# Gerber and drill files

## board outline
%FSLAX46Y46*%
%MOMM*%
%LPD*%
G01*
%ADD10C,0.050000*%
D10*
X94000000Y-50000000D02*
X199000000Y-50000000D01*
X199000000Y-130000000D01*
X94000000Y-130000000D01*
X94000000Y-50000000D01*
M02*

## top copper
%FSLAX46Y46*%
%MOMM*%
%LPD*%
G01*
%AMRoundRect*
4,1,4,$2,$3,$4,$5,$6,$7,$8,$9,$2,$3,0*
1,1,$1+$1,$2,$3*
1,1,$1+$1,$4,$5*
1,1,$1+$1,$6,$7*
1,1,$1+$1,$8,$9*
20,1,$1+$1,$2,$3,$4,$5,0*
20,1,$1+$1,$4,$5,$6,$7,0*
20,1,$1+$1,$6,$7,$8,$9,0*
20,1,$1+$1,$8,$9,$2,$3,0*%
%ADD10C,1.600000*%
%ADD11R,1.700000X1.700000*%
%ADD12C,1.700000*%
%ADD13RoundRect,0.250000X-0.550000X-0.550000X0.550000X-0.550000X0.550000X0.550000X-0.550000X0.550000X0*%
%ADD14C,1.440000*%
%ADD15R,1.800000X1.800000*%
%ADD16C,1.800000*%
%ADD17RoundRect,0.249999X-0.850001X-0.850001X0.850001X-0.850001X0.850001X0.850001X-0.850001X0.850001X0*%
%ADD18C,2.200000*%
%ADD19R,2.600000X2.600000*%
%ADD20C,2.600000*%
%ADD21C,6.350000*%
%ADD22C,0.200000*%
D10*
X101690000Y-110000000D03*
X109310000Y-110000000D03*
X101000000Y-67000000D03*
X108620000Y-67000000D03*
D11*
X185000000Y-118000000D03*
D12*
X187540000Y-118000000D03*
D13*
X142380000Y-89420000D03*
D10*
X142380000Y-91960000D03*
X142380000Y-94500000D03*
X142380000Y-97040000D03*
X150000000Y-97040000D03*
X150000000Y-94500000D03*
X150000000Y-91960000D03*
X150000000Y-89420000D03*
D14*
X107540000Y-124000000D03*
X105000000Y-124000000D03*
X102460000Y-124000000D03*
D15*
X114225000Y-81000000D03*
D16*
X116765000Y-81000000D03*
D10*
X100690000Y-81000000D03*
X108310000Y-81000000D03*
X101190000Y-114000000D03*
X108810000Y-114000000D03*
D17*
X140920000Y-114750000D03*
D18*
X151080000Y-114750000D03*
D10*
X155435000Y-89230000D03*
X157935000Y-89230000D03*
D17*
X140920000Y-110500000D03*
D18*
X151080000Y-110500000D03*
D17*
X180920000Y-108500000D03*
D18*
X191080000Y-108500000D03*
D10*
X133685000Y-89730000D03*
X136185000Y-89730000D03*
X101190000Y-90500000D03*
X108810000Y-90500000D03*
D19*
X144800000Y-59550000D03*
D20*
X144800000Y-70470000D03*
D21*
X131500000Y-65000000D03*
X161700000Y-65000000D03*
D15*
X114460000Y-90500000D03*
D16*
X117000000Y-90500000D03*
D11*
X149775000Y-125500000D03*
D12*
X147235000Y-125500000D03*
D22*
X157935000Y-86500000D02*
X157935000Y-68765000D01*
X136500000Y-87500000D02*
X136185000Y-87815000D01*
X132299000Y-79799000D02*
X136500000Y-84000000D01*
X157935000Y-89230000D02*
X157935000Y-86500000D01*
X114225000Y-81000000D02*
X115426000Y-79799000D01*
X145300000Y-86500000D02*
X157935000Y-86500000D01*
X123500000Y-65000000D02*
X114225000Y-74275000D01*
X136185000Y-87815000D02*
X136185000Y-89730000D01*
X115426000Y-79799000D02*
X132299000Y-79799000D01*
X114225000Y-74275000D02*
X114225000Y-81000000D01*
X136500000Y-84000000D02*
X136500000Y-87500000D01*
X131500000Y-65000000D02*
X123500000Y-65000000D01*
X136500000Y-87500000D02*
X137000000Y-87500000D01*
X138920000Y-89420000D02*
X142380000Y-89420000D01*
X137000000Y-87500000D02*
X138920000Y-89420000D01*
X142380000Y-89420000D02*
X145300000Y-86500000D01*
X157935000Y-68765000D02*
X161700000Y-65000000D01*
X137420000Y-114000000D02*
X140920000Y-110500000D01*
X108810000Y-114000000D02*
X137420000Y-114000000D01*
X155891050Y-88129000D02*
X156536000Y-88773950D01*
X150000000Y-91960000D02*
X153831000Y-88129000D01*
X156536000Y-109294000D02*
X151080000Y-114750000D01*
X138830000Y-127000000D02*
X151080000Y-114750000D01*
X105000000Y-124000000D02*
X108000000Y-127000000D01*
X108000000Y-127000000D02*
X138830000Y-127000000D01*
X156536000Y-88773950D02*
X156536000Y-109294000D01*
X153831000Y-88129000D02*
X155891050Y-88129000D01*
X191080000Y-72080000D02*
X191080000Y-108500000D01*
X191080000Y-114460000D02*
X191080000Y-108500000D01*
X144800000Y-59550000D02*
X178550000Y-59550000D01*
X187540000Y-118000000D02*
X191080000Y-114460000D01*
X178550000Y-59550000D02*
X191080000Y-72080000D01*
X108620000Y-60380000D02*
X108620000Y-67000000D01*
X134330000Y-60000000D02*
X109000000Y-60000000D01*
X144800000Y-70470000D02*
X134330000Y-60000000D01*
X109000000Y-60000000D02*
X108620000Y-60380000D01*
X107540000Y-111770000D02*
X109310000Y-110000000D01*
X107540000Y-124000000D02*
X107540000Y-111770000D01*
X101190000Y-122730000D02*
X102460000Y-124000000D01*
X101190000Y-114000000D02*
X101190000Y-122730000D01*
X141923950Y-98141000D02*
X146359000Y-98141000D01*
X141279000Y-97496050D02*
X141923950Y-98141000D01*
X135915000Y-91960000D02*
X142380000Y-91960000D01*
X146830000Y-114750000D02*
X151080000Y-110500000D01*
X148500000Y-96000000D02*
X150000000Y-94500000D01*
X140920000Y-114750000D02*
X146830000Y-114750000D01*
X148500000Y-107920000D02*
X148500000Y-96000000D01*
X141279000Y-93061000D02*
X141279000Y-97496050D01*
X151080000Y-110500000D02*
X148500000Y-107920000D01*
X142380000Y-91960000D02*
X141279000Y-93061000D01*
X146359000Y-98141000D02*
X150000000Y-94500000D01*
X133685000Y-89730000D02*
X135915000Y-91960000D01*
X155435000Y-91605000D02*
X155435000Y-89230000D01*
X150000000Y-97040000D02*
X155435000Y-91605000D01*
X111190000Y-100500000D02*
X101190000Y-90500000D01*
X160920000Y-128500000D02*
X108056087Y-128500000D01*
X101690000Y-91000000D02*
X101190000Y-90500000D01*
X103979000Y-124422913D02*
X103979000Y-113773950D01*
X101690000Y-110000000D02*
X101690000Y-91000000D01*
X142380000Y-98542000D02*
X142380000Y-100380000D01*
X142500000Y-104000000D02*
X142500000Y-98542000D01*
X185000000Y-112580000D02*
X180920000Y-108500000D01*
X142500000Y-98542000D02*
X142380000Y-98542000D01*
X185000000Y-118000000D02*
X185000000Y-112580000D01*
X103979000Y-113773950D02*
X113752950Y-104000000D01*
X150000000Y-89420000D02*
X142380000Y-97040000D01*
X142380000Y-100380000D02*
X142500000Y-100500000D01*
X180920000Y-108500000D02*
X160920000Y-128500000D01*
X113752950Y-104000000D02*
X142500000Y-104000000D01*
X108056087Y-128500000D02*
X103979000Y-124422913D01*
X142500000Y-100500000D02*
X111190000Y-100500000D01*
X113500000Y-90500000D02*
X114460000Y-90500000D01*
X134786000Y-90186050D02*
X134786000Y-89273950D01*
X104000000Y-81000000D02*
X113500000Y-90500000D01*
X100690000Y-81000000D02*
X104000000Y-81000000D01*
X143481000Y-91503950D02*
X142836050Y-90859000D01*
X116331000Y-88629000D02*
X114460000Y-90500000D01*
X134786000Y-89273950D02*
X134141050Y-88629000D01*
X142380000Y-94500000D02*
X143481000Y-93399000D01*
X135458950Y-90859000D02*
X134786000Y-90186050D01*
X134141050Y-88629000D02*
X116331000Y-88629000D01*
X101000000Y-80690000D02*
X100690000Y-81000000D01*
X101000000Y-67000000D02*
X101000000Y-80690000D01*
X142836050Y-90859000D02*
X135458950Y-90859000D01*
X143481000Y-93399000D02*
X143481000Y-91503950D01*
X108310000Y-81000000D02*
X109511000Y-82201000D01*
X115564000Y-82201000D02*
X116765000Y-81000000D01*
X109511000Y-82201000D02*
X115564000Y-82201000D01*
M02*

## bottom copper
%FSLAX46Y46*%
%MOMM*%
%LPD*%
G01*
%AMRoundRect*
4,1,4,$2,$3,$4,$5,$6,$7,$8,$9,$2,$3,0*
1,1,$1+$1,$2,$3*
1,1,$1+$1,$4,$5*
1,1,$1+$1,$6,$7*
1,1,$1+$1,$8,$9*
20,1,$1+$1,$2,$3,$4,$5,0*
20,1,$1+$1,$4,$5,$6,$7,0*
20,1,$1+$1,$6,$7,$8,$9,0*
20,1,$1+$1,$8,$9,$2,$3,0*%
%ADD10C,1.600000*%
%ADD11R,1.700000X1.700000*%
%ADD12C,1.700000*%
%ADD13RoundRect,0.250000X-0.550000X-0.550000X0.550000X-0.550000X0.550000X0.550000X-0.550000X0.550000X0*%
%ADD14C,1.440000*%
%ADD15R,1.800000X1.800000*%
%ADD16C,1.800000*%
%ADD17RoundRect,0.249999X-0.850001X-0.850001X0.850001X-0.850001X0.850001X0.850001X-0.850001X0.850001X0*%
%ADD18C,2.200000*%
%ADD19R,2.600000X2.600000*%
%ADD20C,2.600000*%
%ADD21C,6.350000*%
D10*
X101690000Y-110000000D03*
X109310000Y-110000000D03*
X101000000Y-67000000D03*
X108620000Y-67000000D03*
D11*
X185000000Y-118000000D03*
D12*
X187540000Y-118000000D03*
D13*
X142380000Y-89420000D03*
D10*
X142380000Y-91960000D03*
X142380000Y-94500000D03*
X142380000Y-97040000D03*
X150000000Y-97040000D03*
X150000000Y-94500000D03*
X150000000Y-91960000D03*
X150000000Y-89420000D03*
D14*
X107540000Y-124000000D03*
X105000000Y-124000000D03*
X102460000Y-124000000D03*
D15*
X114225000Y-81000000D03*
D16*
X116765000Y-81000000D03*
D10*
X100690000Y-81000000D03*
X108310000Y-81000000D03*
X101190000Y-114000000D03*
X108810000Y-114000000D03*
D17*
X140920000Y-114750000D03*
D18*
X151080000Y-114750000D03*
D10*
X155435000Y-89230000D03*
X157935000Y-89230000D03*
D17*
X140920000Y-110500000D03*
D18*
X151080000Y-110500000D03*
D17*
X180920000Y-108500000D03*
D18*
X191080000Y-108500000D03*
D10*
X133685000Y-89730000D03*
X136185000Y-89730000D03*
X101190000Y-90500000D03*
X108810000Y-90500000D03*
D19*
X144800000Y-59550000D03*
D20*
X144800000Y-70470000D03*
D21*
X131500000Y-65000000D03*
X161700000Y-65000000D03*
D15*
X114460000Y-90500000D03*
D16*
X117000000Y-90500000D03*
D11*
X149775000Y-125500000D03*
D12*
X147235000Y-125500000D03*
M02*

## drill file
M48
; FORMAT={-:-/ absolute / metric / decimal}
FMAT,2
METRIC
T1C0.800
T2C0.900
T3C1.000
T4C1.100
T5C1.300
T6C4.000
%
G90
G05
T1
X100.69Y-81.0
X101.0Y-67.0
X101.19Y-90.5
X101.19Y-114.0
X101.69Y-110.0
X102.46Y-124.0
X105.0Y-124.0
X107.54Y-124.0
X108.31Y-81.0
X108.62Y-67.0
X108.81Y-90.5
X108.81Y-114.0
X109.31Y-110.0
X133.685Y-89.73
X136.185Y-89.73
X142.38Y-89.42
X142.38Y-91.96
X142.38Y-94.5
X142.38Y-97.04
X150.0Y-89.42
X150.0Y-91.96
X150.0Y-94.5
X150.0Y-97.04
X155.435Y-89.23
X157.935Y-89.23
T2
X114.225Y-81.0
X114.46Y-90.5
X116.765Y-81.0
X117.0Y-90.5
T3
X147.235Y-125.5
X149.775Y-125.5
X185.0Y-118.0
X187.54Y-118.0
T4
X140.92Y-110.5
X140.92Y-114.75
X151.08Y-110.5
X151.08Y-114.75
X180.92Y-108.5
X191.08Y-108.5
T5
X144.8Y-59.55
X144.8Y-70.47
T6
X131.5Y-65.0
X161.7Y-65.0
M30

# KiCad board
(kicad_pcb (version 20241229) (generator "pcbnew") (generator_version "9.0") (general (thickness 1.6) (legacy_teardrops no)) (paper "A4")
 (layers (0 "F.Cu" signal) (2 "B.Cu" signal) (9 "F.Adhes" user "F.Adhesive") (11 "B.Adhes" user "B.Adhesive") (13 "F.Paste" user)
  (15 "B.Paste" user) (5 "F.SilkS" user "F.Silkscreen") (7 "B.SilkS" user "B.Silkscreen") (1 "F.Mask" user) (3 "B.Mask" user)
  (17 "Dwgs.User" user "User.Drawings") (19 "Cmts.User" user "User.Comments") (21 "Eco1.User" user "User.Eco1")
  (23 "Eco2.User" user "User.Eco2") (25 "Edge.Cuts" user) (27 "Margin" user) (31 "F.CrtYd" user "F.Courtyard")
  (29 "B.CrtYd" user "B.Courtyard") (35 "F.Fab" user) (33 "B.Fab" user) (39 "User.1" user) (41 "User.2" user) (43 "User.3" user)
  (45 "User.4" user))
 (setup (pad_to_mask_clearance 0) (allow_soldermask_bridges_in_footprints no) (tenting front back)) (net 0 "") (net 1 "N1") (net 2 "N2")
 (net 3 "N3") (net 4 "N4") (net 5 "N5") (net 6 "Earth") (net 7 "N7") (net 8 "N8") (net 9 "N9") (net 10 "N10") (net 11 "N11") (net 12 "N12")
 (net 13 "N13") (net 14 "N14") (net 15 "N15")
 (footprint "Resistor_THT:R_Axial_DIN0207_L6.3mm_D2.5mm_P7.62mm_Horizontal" (layer "F.Cu") (at 101.69 110)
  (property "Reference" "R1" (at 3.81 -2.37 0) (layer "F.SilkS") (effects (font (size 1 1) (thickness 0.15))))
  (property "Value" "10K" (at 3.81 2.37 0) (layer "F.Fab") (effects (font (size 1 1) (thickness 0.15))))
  (pad "1" thru_hole circle (at 0 0) (size 1.6 1.6) (drill 0.8) (layers "*.Cu" "*.Mask") (remove_unused_layers no) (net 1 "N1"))
  (pad "2" thru_hole circle (at 7.62 0) (size 1.6 1.6) (drill 0.8) (layers "*.Cu" "*.Mask") (remove_unused_layers no) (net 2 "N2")))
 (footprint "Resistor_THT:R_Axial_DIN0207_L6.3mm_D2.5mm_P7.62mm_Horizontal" (layer "F.Cu") (at 101 67)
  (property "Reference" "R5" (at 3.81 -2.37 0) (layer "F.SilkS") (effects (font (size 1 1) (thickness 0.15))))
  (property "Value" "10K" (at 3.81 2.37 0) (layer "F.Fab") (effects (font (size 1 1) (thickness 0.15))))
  (pad "1" thru_hole circle (at 0 0) (size 1.6 1.6) (drill 0.8) (layers "*.Cu" "*.Mask") (remove_unused_layers no) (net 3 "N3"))
  (pad "2" thru_hole circle (at 7.62 0) (size 1.6 1.6) (drill 0.8) (layers "*.Cu" "*.Mask") (remove_unused_layers no) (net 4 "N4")))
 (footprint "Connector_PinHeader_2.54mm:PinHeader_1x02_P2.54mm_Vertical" (layer "F.Cu") (at 185 118 90)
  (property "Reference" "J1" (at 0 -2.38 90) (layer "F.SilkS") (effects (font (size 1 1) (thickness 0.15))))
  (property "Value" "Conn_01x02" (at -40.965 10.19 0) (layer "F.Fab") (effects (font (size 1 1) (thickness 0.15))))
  (pad "1" thru_hole rect (at 0 0 90) (size 1.7 1.7) (drill 1) (layers "*.Cu" "*.Mask") (remove_unused_layers no) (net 1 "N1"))
  (pad "2" thru_hole circle (at 0 2.54 90) (size 1.7 1.7) (drill 1) (layers "*.Cu" "*.Mask") (remove_unused_layers no) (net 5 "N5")))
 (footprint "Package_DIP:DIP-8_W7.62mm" (layer "F.Cu") (at 142.38 89.42)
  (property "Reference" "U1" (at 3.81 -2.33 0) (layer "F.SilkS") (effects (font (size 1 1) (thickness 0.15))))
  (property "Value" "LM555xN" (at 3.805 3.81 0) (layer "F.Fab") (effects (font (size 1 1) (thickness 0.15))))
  (pad "1" thru_hole roundrect (at 0 0) (size 1.6 1.6) (drill 0.8) (layers "*.Cu" "*.Mask") (remove_unused_layers no)
   (roundrect_rratio 0.15625) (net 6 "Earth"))
  (pad "2" thru_hole circle (at 0 2.54) (size 1.6 1.6) (drill 0.8) (layers "*.Cu" "*.Mask") (remove_unused_layers no) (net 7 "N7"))
  (pad "3" thru_hole circle (at 0 5.08) (size 1.6 1.6) (drill 0.8) (layers "*.Cu" "*.Mask") (remove_unused_layers no) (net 3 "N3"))
  (pad "4" thru_hole circle (at 0 7.62) (size 1.6 1.6) (drill 0.8) (layers "*.Cu" "*.Mask") (remove_unused_layers no) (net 1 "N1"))
  (pad "5" thru_hole circle (at 7.62 7.62) (size 1.6 1.6) (drill 0.8) (layers "*.Cu" "*.Mask") (remove_unused_layers no) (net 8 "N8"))
  (pad "6" thru_hole circle (at 7.62 5.08) (size 1.6 1.6) (drill 0.8) (layers "*.Cu" "*.Mask") (remove_unused_layers no) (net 7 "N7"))
  (pad "7" thru_hole circle (at 7.62 2.54) (size 1.6 1.6) (drill 0.8) (layers "*.Cu" "*.Mask") (remove_unused_layers no) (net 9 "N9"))
  (pad "8" thru_hole circle (at 7.62 0) (size 1.6 1.6) (drill 0.8) (layers "*.Cu" "*.Mask") (remove_unused_layers no) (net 1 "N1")))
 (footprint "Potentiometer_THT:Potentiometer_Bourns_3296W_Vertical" (layer "F.Cu") (at 107.54 124)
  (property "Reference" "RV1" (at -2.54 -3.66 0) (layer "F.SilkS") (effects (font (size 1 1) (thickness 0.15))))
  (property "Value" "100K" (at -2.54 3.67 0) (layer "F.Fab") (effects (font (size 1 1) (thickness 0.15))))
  (pad "1" thru_hole circle (at 0 0) (size 1.44 1.44) (drill 0.8) (layers "*.Cu" "*.Mask") (remove_unused_layers no) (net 2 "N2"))
  (pad "2" thru_hole circle (at -2.54 0) (size 1.44 1.44) (drill 0.8) (layers "*.Cu" "*.Mask") (remove_unused_layers no) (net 9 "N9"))
  (pad "3" thru_hole circle (at -5.08 0) (size 1.44 1.44) (drill 0.8) (layers "*.Cu" "*.Mask") (remove_unused_layers no) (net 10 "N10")))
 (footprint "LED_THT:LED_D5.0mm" (layer "F.Cu") (at 114.225 81)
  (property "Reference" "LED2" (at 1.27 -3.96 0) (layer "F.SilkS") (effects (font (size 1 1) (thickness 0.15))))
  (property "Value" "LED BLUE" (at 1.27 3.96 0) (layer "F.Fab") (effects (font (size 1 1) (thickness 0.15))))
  (pad "1" thru_hole rect (at 0 0) (size 1.8 1.8) (drill 0.9) (layers "*.Cu" "*.Mask") (remove_unused_layers no) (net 6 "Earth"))
  (pad "2" thru_hole circle (at 2.54 0) (size 1.8 1.8) (drill 0.9) (layers "*.Cu" "*.Mask") (remove_unused_layers no) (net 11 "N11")))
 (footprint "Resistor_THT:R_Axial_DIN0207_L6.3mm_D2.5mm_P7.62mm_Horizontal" (layer "F.Cu") (at 100.69 81)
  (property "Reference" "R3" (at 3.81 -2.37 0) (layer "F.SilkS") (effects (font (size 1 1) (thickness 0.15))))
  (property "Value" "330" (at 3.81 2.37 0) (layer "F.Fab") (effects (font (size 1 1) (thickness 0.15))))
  (pad "1" thru_hole circle (at 0 0) (size 1.6 1.6) (drill 0.8) (layers "*.Cu" "*.Mask") (remove_unused_layers no) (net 3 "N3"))
  (pad "2" thru_hole circle (at 7.62 0) (size 1.6 1.6) (drill 0.8) (layers "*.Cu" "*.Mask") (remove_unused_layers no) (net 11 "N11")))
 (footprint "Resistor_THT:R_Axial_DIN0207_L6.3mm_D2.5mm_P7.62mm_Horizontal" (layer "F.Cu") (at 101.19 114)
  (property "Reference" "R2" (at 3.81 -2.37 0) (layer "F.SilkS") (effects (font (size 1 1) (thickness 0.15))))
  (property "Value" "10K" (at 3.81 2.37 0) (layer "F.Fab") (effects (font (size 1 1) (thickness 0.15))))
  (pad "1" thru_hole circle (at 0 0) (size 1.6 1.6) (drill 0.8) (layers "*.Cu" "*.Mask") (remove_unused_layers no) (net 10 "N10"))
  (pad "2" thru_hole circle (at 7.62 0) (size 1.6 1.6) (drill 0.8) (layers "*.Cu" "*.Mask") (remove_unused_layers no) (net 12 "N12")))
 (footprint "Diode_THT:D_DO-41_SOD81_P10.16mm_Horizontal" (layer "F.Cu") (at 140.92 114.75)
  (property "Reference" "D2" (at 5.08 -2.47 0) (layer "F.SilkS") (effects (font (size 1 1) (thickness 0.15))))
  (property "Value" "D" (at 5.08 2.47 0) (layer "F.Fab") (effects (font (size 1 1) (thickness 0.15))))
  (pad "1" thru_hole roundrect (at 0 0) (size 2.2 2.2) (drill 1.1) (layers "*.Cu" "*.Mask") (remove_unused_layers no)
   (roundrect_rratio 0.113636) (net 7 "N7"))
  (pad "2" thru_hole circle (at 10.16 0) (size 2.2 2.2) (drill 1.1) (layers "*.Cu" "*.Mask") (remove_unused_layers no) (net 9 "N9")))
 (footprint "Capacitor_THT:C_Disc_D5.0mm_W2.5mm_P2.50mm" (layer "F.Cu") (at 155.435 89.23)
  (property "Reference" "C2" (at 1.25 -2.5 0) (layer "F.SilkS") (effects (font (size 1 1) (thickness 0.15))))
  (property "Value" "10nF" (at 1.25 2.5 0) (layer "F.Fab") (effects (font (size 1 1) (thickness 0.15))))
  (pad "1" thru_hole circle (at 0 0) (size 1.6 1.6) (drill 0.8) (layers "*.Cu" "*.Mask") (remove_unused_layers no) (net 8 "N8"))
  (pad "2" thru_hole circle (at 2.5 0) (size 1.6 1.6) (drill 0.8) (layers "*.Cu" "*.Mask") (remove_unused_layers no) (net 6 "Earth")))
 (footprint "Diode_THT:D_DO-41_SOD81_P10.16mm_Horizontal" (layer "F.Cu") (at 140.92 110.5)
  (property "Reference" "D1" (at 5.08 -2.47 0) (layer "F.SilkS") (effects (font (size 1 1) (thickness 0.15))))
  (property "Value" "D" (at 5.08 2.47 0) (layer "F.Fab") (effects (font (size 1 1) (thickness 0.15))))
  (pad "1" thru_hole roundrect (at 0 0) (size 2.2 2.2) (drill 1.1) (layers "*.Cu" "*.Mask") (remove_unused_layers no)
   (roundrect_rratio 0.113636) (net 12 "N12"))
  (pad "2" thru_hole circle (at 10.16 0) (size 2.2 2.2) (drill 1.1) (layers "*.Cu" "*.Mask") (remove_unused_layers no) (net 7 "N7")))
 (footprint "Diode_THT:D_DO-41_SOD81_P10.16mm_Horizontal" (layer "F.Cu") (at 180.92 108.5)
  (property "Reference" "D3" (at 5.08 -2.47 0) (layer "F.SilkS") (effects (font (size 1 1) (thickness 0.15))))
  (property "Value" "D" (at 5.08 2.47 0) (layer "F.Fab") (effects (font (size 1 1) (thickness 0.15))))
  (pad "1" thru_hole roundrect (at 0 0) (size 2.2 2.2) (drill 1.1) (layers "*.Cu" "*.Mask") (remove_unused_layers no)
   (roundrect_rratio 0.113636) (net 1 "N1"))
  (pad "2" thru_hole circle (at 10.16 0) (size 2.2 2.2) (drill 1.1) (layers "*.Cu" "*.Mask") (remove_unused_layers no) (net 5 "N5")))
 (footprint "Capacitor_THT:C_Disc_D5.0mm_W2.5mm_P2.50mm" (layer "F.Cu") (at 133.685 89.73)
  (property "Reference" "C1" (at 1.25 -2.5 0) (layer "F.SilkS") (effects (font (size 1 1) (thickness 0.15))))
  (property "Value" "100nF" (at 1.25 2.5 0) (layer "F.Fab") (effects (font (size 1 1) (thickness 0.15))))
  (pad "1" thru_hole circle (at 0 0) (size 1.6 1.6) (drill 0.8) (layers "*.Cu" "*.Mask") (remove_unused_layers no) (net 7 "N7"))
  (pad "2" thru_hole circle (at 2.5 0) (size 1.6 1.6) (drill 0.8) (layers "*.Cu" "*.Mask") (remove_unused_layers no) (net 6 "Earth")))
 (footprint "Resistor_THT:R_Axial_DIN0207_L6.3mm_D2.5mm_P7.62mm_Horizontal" (layer "F.Cu") (at 101.19 90.5)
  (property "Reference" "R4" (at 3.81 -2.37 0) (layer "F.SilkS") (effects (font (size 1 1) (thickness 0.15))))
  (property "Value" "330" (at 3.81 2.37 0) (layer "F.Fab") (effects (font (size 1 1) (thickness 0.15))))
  (pad "1" thru_hole circle (at 0 0) (size 1.6 1.6) (drill 0.8) (layers "*.Cu" "*.Mask") (remove_unused_layers no) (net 1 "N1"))
  (pad "2" thru_hole circle (at 7.62 0) (size 1.6 1.6) (drill 0.8) (layers "*.Cu" "*.Mask") (remove_unused_layers no) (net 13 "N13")))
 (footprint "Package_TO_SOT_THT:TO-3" (layer "F.Cu") (at 144.8 59.55)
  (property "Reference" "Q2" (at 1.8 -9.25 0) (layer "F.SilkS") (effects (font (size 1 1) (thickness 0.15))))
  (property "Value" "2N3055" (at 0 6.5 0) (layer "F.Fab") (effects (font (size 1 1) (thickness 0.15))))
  (pad "1" thru_hole rect (at 0 0) (size 2.6 2.6) (drill 1.3) (layers "*.Cu" "*.Mask") (remove_unused_layers no) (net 5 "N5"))
  (pad "2" thru_hole circle (at 0 10.92) (size 2.6 2.6) (drill 1.3) (layers "*.Cu" "*.Mask") (remove_unused_layers no) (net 4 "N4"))
  (pad "3" thru_hole circle (at -13.3 5.45) (size 6.35 6.35) (drill 4) (layers "*.Cu" "*.Mask") (remove_unused_layers no) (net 6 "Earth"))
  (pad "3" thru_hole circle (at 16.9 5.45) (size 6.35 6.35) (drill 4) (layers "*.Cu" "*.Mask") (remove_unused_layers no) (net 6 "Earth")))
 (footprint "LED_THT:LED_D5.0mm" (layer "F.Cu") (at 114.46 90.5)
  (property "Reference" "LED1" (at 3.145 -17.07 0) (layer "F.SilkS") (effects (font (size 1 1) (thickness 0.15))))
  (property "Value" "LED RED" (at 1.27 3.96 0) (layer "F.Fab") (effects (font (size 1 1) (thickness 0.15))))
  (pad "1" thru_hole rect (at 0 0) (size 1.8 1.8) (drill 0.9) (layers "*.Cu" "*.Mask") (remove_unused_layers no) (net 3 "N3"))
  (pad "2" thru_hole circle (at 2.54 0) (size 1.8 1.8) (drill 0.9) (layers "*.Cu" "*.Mask") (remove_unused_layers no) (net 13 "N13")))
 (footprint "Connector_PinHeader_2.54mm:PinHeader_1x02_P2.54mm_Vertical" (layer "F.Cu") (at 149.775 125.5 -90)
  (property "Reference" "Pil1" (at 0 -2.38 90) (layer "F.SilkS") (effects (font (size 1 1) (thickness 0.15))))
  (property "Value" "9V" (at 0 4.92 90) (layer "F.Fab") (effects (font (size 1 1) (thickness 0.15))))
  (pad "1" thru_hole rect (at 0 0 270) (size 1.7 1.7) (drill 1) (layers "*.Cu" "*.Mask") (remove_unused_layers no) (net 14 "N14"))
  (pad "2" thru_hole circle (at 0 2.54 270) (size 1.7 1.7) (drill 1) (layers "*.Cu" "*.Mask") (remove_unused_layers no) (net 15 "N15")))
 (gr_rect (start 94 50) (end 199 130) (stroke (width 0.05) (type default)) (fill no) (layer "Edge.Cuts"))
 (segment (start 157.935 86.5) (end 157.935 68.765) (width 0.2) (layer "F.Cu") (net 6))
 (segment (start 136.5 87.5) (end 136.185 87.815) (width 0.2) (layer "F.Cu") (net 6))
 (segment (start 132.299 79.799) (end 136.5 84) (width 0.2) (layer "F.Cu") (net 6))
 (segment (start 157.935 89.23) (end 157.935 86.5) (width 0.2) (layer "F.Cu") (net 6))
 (segment (start 114.225 81) (end 115.426 79.799) (width 0.2) (layer "F.Cu") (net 6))
 (segment (start 145.3 86.5) (end 157.935 86.5) (width 0.2) (layer "F.Cu") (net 6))
 (segment (start 123.5 65) (end 114.225 74.275) (width 0.2) (layer "F.Cu") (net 6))
 (segment (start 136.185 87.815) (end 136.185 89.73) (width 0.2) (layer "F.Cu") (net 6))
 (segment (start 115.426 79.799) (end 132.299 79.799) (width 0.2) (layer "F.Cu") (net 6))
 (segment (start 114.225 74.275) (end 114.225 81) (width 0.2) (layer "F.Cu") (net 6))
 (segment (start 136.5 84) (end 136.5 87.5) (width 0.2) (layer "F.Cu") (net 6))
 (segment (start 131.5 65) (end 123.5 65) (width 0.2) (layer "F.Cu") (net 6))
 (segment (start 136.5 87.5) (end 137 87.5) (width 0.2) (layer "F.Cu") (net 6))
 (segment (start 138.92 89.42) (end 142.38 89.42) (width 0.2) (layer "F.Cu") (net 6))
 (segment (start 137 87.5) (end 138.92 89.42) (width 0.2) (layer "F.Cu") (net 6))
 (segment (start 142.38 89.42) (end 145.3 86.5) (width 0.2) (layer "F.Cu") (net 6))
 (segment (start 157.935 68.765) (end 161.7 65) (width 0.2) (layer "F.Cu") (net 6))
 (segment (start 137.42 114) (end 140.92 110.5) (width 0.2) (layer "F.Cu") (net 12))
 (segment (start 108.81 114) (end 137.42 114) (width 0.2) (layer "F.Cu") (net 12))
 (segment (start 155.89105 88.129) (end 156.536 88.77395) (width 0.2) (layer "F.Cu") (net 9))
 (segment (start 150 91.96) (end 153.831 88.129) (width 0.2) (layer "F.Cu") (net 9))
 (segment (start 156.536 109.294) (end 151.08 114.75) (width 0.2) (layer "F.Cu") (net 9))
 (segment (start 138.83 127) (end 151.08 114.75) (width 0.2) (layer "F.Cu") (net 9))
 (segment (start 105 124) (end 108 127) (width 0.2) (layer "F.Cu") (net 9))
 (segment (start 108 127) (end 138.83 127) (width 0.2) (layer "F.Cu") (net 9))
 (segment (start 156.536 88.77395) (end 156.536 109.294) (width 0.2) (layer "F.Cu") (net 9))
 (segment (start 153.831 88.129) (end 155.89105 88.129) (width 0.2) (layer "F.Cu") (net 9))
 (segment (start 191.08 72.08) (end 191.08 108.5) (width 0.2) (layer "F.Cu") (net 5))
 (segment (start 191.08 114.46) (end 191.08 108.5) (width 0.2) (layer "F.Cu") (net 5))
 (segment (start 144.8 59.55) (end 178.55 59.55) (width 0.2) (layer "F.Cu") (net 5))
 (segment (start 187.54 118) (end 191.08 114.46) (width 0.2) (layer "F.Cu") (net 5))
 (segment (start 178.55 59.55) (end 191.08 72.08) (width 0.2) (layer "F.Cu") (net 5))
 (segment (start 108.62 60.38) (end 108.62 67) (width 0.2) (layer "F.Cu") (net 4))
 (segment (start 134.33 60) (end 109 60) (width 0.2) (layer "F.Cu") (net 4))
 (segment (start 144.8 70.47) (end 134.33 60) (width 0.2) (layer "F.Cu") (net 4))
 (segment (start 109 60) (end 108.62 60.38) (width 0.2) (layer "F.Cu") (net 4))
 (segment (start 107.54 111.77) (end 109.31 110) (width 0.2) (layer "F.Cu") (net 2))
 (segment (start 107.54 124) (end 107.54 111.77) (width 0.2) (layer "F.Cu") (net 2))
 (segment (start 101.19 122.73) (end 102.46 124) (width 0.2) (layer "F.Cu") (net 10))
 (segment (start 101.19 114) (end 101.19 122.73) (width 0.2) (layer "F.Cu") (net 10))
 (segment (start 141.92395 98.141) (end 146.359 98.141) (width 0.2) (layer "F.Cu") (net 7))
 (segment (start 141.279 97.49605) (end 141.92395 98.141) (width 0.2) (layer "F.Cu") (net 7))
 (segment (start 135.915 91.96) (end 142.38 91.96) (width 0.2) (layer "F.Cu") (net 7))
 (segment (start 146.83 114.75) (end 151.08 110.5) (width 0.2) (layer "F.Cu") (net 7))
 (segment (start 148.5 96) (end 150 94.5) (width 0.2) (layer "F.Cu") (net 7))
 (segment (start 140.92 114.75) (end 146.83 114.75) (width 0.2) (layer "F.Cu") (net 7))
 (segment (start 148.5 107.92) (end 148.5 96) (width 0.2) (layer "F.Cu") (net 7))
 (segment (start 141.279 93.061) (end 141.279 97.49605) (width 0.2) (layer "F.Cu") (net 7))
 (segment (start 151.08 110.5) (end 148.5 107.92) (width 0.2) (layer "F.Cu") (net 7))
 (segment (start 142.38 91.96) (end 141.279 93.061) (width 0.2) (layer "F.Cu") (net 7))
 (segment (start 146.359 98.141) (end 150 94.5) (width 0.2) (layer "F.Cu") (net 7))
 (segment (start 133.685 89.73) (end 135.915 91.96) (width 0.2) (layer "F.Cu") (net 7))
 (segment (start 155.435 91.605) (end 155.435 89.23) (width 0.2) (layer "F.Cu") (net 8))
 (segment (start 150 97.04) (end 155.435 91.605) (width 0.2) (layer "F.Cu") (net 8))
 (segment (start 111.19 100.5) (end 101.19 90.5) (width 0.2) (layer "F.Cu") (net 1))
 (segment (start 160.92 128.5) (end 108.056087 128.5) (width 0.2) (layer "F.Cu") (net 1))
 (segment (start 101.69 91) (end 101.19 90.5) (width 0.2) (layer "F.Cu") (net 1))
 (segment (start 103.979 124.422913) (end 103.979 113.77395) (width 0.2) (layer "F.Cu") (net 1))
 (segment (start 101.69 110) (end 101.69 91) (width 0.2) (layer "F.Cu") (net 1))
 (segment (start 142.38 98.542) (end 142.38 100.38) (width 0.2) (layer "F.Cu") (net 1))
 (segment (start 142.5 104) (end 142.5 98.542) (width 0.2) (layer "F.Cu") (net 1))
 (segment (start 185 112.58) (end 180.92 108.5) (width 0.2) (layer "F.Cu") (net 1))
 (segment (start 142.5 98.542) (end 142.38 98.542) (width 0.2) (layer "F.Cu") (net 1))
 (segment (start 185 118) (end 185 112.58) (width 0.2) (layer "F.Cu") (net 1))
 (segment (start 103.979 113.77395) (end 113.75295 104) (width 0.2) (layer "F.Cu") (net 1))
 (segment (start 150 89.42) (end 142.38 97.04) (width 0.2) (layer "F.Cu") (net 1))
 (segment (start 142.38 100.38) (end 142.5 100.5) (width 0.2) (layer "F.Cu") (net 1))
 (segment (start 180.92 108.5) (end 160.92 128.5) (width 0.2) (layer "F.Cu") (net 1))
 (segment (start 113.75295 104) (end 142.5 104) (width 0.2) (layer "F.Cu") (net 1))
 (segment (start 108.056087 128.5) (end 103.979 124.422913) (width 0.2) (layer "F.Cu") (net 1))
 (segment (start 142.5 100.5) (end 111.19 100.5) (width 0.2) (layer "F.Cu") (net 1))
 (segment (start 113.5 90.5) (end 114.46 90.5) (width 0.2) (layer "F.Cu") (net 3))
 (segment (start 134.786 90.18605) (end 134.786 89.27395) (width 0.2) (layer "F.Cu") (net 3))
 (segment (start 104 81) (end 113.5 90.5) (width 0.2) (layer "F.Cu") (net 3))
 (segment (start 100.69 81) (end 104 81) (width 0.2) (layer "F.Cu") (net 3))
 (segment (start 143.481 91.50395) (end 142.83605 90.859) (width 0.2) (layer "F.Cu") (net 3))
 (segment (start 116.331 88.629) (end 114.46 90.5) (width 0.2) (layer "F.Cu") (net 3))
 (segment (start 134.786 89.27395) (end 134.14105 88.629) (width 0.2) (layer "F.Cu") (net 3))
 (segment (start 142.38 94.5) (end 143.481 93.399) (width 0.2) (layer "F.Cu") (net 3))
 (segment (start 135.45895 90.859) (end 134.786 90.18605) (width 0.2) (layer "F.Cu") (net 3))
 (segment (start 134.14105 88.629) (end 116.331 88.629) (width 0.2) (layer "F.Cu") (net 3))
 (segment (start 101 80.69) (end 100.69 81) (width 0.2) (layer "F.Cu") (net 3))
 (segment (start 101 67) (end 101 80.69) (width 0.2) (layer "F.Cu") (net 3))
 (segment (start 142.83605 90.859) (end 135.45895 90.859) (width 0.2) (layer "F.Cu") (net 3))
 (segment (start 143.481 93.399) (end 143.481 91.50395) (width 0.2) (layer "F.Cu") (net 3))
 (segment (start 108.31 81) (end 109.511 82.201) (width 0.2) (layer "F.Cu") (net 11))
 (segment (start 115.564 82.201) (end 116.765 81) (width 0.2) (layer "F.Cu") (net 11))
 (segment (start 109.511 82.201) (end 115.564 82.201) (width 0.2) (layer "F.Cu") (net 11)))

